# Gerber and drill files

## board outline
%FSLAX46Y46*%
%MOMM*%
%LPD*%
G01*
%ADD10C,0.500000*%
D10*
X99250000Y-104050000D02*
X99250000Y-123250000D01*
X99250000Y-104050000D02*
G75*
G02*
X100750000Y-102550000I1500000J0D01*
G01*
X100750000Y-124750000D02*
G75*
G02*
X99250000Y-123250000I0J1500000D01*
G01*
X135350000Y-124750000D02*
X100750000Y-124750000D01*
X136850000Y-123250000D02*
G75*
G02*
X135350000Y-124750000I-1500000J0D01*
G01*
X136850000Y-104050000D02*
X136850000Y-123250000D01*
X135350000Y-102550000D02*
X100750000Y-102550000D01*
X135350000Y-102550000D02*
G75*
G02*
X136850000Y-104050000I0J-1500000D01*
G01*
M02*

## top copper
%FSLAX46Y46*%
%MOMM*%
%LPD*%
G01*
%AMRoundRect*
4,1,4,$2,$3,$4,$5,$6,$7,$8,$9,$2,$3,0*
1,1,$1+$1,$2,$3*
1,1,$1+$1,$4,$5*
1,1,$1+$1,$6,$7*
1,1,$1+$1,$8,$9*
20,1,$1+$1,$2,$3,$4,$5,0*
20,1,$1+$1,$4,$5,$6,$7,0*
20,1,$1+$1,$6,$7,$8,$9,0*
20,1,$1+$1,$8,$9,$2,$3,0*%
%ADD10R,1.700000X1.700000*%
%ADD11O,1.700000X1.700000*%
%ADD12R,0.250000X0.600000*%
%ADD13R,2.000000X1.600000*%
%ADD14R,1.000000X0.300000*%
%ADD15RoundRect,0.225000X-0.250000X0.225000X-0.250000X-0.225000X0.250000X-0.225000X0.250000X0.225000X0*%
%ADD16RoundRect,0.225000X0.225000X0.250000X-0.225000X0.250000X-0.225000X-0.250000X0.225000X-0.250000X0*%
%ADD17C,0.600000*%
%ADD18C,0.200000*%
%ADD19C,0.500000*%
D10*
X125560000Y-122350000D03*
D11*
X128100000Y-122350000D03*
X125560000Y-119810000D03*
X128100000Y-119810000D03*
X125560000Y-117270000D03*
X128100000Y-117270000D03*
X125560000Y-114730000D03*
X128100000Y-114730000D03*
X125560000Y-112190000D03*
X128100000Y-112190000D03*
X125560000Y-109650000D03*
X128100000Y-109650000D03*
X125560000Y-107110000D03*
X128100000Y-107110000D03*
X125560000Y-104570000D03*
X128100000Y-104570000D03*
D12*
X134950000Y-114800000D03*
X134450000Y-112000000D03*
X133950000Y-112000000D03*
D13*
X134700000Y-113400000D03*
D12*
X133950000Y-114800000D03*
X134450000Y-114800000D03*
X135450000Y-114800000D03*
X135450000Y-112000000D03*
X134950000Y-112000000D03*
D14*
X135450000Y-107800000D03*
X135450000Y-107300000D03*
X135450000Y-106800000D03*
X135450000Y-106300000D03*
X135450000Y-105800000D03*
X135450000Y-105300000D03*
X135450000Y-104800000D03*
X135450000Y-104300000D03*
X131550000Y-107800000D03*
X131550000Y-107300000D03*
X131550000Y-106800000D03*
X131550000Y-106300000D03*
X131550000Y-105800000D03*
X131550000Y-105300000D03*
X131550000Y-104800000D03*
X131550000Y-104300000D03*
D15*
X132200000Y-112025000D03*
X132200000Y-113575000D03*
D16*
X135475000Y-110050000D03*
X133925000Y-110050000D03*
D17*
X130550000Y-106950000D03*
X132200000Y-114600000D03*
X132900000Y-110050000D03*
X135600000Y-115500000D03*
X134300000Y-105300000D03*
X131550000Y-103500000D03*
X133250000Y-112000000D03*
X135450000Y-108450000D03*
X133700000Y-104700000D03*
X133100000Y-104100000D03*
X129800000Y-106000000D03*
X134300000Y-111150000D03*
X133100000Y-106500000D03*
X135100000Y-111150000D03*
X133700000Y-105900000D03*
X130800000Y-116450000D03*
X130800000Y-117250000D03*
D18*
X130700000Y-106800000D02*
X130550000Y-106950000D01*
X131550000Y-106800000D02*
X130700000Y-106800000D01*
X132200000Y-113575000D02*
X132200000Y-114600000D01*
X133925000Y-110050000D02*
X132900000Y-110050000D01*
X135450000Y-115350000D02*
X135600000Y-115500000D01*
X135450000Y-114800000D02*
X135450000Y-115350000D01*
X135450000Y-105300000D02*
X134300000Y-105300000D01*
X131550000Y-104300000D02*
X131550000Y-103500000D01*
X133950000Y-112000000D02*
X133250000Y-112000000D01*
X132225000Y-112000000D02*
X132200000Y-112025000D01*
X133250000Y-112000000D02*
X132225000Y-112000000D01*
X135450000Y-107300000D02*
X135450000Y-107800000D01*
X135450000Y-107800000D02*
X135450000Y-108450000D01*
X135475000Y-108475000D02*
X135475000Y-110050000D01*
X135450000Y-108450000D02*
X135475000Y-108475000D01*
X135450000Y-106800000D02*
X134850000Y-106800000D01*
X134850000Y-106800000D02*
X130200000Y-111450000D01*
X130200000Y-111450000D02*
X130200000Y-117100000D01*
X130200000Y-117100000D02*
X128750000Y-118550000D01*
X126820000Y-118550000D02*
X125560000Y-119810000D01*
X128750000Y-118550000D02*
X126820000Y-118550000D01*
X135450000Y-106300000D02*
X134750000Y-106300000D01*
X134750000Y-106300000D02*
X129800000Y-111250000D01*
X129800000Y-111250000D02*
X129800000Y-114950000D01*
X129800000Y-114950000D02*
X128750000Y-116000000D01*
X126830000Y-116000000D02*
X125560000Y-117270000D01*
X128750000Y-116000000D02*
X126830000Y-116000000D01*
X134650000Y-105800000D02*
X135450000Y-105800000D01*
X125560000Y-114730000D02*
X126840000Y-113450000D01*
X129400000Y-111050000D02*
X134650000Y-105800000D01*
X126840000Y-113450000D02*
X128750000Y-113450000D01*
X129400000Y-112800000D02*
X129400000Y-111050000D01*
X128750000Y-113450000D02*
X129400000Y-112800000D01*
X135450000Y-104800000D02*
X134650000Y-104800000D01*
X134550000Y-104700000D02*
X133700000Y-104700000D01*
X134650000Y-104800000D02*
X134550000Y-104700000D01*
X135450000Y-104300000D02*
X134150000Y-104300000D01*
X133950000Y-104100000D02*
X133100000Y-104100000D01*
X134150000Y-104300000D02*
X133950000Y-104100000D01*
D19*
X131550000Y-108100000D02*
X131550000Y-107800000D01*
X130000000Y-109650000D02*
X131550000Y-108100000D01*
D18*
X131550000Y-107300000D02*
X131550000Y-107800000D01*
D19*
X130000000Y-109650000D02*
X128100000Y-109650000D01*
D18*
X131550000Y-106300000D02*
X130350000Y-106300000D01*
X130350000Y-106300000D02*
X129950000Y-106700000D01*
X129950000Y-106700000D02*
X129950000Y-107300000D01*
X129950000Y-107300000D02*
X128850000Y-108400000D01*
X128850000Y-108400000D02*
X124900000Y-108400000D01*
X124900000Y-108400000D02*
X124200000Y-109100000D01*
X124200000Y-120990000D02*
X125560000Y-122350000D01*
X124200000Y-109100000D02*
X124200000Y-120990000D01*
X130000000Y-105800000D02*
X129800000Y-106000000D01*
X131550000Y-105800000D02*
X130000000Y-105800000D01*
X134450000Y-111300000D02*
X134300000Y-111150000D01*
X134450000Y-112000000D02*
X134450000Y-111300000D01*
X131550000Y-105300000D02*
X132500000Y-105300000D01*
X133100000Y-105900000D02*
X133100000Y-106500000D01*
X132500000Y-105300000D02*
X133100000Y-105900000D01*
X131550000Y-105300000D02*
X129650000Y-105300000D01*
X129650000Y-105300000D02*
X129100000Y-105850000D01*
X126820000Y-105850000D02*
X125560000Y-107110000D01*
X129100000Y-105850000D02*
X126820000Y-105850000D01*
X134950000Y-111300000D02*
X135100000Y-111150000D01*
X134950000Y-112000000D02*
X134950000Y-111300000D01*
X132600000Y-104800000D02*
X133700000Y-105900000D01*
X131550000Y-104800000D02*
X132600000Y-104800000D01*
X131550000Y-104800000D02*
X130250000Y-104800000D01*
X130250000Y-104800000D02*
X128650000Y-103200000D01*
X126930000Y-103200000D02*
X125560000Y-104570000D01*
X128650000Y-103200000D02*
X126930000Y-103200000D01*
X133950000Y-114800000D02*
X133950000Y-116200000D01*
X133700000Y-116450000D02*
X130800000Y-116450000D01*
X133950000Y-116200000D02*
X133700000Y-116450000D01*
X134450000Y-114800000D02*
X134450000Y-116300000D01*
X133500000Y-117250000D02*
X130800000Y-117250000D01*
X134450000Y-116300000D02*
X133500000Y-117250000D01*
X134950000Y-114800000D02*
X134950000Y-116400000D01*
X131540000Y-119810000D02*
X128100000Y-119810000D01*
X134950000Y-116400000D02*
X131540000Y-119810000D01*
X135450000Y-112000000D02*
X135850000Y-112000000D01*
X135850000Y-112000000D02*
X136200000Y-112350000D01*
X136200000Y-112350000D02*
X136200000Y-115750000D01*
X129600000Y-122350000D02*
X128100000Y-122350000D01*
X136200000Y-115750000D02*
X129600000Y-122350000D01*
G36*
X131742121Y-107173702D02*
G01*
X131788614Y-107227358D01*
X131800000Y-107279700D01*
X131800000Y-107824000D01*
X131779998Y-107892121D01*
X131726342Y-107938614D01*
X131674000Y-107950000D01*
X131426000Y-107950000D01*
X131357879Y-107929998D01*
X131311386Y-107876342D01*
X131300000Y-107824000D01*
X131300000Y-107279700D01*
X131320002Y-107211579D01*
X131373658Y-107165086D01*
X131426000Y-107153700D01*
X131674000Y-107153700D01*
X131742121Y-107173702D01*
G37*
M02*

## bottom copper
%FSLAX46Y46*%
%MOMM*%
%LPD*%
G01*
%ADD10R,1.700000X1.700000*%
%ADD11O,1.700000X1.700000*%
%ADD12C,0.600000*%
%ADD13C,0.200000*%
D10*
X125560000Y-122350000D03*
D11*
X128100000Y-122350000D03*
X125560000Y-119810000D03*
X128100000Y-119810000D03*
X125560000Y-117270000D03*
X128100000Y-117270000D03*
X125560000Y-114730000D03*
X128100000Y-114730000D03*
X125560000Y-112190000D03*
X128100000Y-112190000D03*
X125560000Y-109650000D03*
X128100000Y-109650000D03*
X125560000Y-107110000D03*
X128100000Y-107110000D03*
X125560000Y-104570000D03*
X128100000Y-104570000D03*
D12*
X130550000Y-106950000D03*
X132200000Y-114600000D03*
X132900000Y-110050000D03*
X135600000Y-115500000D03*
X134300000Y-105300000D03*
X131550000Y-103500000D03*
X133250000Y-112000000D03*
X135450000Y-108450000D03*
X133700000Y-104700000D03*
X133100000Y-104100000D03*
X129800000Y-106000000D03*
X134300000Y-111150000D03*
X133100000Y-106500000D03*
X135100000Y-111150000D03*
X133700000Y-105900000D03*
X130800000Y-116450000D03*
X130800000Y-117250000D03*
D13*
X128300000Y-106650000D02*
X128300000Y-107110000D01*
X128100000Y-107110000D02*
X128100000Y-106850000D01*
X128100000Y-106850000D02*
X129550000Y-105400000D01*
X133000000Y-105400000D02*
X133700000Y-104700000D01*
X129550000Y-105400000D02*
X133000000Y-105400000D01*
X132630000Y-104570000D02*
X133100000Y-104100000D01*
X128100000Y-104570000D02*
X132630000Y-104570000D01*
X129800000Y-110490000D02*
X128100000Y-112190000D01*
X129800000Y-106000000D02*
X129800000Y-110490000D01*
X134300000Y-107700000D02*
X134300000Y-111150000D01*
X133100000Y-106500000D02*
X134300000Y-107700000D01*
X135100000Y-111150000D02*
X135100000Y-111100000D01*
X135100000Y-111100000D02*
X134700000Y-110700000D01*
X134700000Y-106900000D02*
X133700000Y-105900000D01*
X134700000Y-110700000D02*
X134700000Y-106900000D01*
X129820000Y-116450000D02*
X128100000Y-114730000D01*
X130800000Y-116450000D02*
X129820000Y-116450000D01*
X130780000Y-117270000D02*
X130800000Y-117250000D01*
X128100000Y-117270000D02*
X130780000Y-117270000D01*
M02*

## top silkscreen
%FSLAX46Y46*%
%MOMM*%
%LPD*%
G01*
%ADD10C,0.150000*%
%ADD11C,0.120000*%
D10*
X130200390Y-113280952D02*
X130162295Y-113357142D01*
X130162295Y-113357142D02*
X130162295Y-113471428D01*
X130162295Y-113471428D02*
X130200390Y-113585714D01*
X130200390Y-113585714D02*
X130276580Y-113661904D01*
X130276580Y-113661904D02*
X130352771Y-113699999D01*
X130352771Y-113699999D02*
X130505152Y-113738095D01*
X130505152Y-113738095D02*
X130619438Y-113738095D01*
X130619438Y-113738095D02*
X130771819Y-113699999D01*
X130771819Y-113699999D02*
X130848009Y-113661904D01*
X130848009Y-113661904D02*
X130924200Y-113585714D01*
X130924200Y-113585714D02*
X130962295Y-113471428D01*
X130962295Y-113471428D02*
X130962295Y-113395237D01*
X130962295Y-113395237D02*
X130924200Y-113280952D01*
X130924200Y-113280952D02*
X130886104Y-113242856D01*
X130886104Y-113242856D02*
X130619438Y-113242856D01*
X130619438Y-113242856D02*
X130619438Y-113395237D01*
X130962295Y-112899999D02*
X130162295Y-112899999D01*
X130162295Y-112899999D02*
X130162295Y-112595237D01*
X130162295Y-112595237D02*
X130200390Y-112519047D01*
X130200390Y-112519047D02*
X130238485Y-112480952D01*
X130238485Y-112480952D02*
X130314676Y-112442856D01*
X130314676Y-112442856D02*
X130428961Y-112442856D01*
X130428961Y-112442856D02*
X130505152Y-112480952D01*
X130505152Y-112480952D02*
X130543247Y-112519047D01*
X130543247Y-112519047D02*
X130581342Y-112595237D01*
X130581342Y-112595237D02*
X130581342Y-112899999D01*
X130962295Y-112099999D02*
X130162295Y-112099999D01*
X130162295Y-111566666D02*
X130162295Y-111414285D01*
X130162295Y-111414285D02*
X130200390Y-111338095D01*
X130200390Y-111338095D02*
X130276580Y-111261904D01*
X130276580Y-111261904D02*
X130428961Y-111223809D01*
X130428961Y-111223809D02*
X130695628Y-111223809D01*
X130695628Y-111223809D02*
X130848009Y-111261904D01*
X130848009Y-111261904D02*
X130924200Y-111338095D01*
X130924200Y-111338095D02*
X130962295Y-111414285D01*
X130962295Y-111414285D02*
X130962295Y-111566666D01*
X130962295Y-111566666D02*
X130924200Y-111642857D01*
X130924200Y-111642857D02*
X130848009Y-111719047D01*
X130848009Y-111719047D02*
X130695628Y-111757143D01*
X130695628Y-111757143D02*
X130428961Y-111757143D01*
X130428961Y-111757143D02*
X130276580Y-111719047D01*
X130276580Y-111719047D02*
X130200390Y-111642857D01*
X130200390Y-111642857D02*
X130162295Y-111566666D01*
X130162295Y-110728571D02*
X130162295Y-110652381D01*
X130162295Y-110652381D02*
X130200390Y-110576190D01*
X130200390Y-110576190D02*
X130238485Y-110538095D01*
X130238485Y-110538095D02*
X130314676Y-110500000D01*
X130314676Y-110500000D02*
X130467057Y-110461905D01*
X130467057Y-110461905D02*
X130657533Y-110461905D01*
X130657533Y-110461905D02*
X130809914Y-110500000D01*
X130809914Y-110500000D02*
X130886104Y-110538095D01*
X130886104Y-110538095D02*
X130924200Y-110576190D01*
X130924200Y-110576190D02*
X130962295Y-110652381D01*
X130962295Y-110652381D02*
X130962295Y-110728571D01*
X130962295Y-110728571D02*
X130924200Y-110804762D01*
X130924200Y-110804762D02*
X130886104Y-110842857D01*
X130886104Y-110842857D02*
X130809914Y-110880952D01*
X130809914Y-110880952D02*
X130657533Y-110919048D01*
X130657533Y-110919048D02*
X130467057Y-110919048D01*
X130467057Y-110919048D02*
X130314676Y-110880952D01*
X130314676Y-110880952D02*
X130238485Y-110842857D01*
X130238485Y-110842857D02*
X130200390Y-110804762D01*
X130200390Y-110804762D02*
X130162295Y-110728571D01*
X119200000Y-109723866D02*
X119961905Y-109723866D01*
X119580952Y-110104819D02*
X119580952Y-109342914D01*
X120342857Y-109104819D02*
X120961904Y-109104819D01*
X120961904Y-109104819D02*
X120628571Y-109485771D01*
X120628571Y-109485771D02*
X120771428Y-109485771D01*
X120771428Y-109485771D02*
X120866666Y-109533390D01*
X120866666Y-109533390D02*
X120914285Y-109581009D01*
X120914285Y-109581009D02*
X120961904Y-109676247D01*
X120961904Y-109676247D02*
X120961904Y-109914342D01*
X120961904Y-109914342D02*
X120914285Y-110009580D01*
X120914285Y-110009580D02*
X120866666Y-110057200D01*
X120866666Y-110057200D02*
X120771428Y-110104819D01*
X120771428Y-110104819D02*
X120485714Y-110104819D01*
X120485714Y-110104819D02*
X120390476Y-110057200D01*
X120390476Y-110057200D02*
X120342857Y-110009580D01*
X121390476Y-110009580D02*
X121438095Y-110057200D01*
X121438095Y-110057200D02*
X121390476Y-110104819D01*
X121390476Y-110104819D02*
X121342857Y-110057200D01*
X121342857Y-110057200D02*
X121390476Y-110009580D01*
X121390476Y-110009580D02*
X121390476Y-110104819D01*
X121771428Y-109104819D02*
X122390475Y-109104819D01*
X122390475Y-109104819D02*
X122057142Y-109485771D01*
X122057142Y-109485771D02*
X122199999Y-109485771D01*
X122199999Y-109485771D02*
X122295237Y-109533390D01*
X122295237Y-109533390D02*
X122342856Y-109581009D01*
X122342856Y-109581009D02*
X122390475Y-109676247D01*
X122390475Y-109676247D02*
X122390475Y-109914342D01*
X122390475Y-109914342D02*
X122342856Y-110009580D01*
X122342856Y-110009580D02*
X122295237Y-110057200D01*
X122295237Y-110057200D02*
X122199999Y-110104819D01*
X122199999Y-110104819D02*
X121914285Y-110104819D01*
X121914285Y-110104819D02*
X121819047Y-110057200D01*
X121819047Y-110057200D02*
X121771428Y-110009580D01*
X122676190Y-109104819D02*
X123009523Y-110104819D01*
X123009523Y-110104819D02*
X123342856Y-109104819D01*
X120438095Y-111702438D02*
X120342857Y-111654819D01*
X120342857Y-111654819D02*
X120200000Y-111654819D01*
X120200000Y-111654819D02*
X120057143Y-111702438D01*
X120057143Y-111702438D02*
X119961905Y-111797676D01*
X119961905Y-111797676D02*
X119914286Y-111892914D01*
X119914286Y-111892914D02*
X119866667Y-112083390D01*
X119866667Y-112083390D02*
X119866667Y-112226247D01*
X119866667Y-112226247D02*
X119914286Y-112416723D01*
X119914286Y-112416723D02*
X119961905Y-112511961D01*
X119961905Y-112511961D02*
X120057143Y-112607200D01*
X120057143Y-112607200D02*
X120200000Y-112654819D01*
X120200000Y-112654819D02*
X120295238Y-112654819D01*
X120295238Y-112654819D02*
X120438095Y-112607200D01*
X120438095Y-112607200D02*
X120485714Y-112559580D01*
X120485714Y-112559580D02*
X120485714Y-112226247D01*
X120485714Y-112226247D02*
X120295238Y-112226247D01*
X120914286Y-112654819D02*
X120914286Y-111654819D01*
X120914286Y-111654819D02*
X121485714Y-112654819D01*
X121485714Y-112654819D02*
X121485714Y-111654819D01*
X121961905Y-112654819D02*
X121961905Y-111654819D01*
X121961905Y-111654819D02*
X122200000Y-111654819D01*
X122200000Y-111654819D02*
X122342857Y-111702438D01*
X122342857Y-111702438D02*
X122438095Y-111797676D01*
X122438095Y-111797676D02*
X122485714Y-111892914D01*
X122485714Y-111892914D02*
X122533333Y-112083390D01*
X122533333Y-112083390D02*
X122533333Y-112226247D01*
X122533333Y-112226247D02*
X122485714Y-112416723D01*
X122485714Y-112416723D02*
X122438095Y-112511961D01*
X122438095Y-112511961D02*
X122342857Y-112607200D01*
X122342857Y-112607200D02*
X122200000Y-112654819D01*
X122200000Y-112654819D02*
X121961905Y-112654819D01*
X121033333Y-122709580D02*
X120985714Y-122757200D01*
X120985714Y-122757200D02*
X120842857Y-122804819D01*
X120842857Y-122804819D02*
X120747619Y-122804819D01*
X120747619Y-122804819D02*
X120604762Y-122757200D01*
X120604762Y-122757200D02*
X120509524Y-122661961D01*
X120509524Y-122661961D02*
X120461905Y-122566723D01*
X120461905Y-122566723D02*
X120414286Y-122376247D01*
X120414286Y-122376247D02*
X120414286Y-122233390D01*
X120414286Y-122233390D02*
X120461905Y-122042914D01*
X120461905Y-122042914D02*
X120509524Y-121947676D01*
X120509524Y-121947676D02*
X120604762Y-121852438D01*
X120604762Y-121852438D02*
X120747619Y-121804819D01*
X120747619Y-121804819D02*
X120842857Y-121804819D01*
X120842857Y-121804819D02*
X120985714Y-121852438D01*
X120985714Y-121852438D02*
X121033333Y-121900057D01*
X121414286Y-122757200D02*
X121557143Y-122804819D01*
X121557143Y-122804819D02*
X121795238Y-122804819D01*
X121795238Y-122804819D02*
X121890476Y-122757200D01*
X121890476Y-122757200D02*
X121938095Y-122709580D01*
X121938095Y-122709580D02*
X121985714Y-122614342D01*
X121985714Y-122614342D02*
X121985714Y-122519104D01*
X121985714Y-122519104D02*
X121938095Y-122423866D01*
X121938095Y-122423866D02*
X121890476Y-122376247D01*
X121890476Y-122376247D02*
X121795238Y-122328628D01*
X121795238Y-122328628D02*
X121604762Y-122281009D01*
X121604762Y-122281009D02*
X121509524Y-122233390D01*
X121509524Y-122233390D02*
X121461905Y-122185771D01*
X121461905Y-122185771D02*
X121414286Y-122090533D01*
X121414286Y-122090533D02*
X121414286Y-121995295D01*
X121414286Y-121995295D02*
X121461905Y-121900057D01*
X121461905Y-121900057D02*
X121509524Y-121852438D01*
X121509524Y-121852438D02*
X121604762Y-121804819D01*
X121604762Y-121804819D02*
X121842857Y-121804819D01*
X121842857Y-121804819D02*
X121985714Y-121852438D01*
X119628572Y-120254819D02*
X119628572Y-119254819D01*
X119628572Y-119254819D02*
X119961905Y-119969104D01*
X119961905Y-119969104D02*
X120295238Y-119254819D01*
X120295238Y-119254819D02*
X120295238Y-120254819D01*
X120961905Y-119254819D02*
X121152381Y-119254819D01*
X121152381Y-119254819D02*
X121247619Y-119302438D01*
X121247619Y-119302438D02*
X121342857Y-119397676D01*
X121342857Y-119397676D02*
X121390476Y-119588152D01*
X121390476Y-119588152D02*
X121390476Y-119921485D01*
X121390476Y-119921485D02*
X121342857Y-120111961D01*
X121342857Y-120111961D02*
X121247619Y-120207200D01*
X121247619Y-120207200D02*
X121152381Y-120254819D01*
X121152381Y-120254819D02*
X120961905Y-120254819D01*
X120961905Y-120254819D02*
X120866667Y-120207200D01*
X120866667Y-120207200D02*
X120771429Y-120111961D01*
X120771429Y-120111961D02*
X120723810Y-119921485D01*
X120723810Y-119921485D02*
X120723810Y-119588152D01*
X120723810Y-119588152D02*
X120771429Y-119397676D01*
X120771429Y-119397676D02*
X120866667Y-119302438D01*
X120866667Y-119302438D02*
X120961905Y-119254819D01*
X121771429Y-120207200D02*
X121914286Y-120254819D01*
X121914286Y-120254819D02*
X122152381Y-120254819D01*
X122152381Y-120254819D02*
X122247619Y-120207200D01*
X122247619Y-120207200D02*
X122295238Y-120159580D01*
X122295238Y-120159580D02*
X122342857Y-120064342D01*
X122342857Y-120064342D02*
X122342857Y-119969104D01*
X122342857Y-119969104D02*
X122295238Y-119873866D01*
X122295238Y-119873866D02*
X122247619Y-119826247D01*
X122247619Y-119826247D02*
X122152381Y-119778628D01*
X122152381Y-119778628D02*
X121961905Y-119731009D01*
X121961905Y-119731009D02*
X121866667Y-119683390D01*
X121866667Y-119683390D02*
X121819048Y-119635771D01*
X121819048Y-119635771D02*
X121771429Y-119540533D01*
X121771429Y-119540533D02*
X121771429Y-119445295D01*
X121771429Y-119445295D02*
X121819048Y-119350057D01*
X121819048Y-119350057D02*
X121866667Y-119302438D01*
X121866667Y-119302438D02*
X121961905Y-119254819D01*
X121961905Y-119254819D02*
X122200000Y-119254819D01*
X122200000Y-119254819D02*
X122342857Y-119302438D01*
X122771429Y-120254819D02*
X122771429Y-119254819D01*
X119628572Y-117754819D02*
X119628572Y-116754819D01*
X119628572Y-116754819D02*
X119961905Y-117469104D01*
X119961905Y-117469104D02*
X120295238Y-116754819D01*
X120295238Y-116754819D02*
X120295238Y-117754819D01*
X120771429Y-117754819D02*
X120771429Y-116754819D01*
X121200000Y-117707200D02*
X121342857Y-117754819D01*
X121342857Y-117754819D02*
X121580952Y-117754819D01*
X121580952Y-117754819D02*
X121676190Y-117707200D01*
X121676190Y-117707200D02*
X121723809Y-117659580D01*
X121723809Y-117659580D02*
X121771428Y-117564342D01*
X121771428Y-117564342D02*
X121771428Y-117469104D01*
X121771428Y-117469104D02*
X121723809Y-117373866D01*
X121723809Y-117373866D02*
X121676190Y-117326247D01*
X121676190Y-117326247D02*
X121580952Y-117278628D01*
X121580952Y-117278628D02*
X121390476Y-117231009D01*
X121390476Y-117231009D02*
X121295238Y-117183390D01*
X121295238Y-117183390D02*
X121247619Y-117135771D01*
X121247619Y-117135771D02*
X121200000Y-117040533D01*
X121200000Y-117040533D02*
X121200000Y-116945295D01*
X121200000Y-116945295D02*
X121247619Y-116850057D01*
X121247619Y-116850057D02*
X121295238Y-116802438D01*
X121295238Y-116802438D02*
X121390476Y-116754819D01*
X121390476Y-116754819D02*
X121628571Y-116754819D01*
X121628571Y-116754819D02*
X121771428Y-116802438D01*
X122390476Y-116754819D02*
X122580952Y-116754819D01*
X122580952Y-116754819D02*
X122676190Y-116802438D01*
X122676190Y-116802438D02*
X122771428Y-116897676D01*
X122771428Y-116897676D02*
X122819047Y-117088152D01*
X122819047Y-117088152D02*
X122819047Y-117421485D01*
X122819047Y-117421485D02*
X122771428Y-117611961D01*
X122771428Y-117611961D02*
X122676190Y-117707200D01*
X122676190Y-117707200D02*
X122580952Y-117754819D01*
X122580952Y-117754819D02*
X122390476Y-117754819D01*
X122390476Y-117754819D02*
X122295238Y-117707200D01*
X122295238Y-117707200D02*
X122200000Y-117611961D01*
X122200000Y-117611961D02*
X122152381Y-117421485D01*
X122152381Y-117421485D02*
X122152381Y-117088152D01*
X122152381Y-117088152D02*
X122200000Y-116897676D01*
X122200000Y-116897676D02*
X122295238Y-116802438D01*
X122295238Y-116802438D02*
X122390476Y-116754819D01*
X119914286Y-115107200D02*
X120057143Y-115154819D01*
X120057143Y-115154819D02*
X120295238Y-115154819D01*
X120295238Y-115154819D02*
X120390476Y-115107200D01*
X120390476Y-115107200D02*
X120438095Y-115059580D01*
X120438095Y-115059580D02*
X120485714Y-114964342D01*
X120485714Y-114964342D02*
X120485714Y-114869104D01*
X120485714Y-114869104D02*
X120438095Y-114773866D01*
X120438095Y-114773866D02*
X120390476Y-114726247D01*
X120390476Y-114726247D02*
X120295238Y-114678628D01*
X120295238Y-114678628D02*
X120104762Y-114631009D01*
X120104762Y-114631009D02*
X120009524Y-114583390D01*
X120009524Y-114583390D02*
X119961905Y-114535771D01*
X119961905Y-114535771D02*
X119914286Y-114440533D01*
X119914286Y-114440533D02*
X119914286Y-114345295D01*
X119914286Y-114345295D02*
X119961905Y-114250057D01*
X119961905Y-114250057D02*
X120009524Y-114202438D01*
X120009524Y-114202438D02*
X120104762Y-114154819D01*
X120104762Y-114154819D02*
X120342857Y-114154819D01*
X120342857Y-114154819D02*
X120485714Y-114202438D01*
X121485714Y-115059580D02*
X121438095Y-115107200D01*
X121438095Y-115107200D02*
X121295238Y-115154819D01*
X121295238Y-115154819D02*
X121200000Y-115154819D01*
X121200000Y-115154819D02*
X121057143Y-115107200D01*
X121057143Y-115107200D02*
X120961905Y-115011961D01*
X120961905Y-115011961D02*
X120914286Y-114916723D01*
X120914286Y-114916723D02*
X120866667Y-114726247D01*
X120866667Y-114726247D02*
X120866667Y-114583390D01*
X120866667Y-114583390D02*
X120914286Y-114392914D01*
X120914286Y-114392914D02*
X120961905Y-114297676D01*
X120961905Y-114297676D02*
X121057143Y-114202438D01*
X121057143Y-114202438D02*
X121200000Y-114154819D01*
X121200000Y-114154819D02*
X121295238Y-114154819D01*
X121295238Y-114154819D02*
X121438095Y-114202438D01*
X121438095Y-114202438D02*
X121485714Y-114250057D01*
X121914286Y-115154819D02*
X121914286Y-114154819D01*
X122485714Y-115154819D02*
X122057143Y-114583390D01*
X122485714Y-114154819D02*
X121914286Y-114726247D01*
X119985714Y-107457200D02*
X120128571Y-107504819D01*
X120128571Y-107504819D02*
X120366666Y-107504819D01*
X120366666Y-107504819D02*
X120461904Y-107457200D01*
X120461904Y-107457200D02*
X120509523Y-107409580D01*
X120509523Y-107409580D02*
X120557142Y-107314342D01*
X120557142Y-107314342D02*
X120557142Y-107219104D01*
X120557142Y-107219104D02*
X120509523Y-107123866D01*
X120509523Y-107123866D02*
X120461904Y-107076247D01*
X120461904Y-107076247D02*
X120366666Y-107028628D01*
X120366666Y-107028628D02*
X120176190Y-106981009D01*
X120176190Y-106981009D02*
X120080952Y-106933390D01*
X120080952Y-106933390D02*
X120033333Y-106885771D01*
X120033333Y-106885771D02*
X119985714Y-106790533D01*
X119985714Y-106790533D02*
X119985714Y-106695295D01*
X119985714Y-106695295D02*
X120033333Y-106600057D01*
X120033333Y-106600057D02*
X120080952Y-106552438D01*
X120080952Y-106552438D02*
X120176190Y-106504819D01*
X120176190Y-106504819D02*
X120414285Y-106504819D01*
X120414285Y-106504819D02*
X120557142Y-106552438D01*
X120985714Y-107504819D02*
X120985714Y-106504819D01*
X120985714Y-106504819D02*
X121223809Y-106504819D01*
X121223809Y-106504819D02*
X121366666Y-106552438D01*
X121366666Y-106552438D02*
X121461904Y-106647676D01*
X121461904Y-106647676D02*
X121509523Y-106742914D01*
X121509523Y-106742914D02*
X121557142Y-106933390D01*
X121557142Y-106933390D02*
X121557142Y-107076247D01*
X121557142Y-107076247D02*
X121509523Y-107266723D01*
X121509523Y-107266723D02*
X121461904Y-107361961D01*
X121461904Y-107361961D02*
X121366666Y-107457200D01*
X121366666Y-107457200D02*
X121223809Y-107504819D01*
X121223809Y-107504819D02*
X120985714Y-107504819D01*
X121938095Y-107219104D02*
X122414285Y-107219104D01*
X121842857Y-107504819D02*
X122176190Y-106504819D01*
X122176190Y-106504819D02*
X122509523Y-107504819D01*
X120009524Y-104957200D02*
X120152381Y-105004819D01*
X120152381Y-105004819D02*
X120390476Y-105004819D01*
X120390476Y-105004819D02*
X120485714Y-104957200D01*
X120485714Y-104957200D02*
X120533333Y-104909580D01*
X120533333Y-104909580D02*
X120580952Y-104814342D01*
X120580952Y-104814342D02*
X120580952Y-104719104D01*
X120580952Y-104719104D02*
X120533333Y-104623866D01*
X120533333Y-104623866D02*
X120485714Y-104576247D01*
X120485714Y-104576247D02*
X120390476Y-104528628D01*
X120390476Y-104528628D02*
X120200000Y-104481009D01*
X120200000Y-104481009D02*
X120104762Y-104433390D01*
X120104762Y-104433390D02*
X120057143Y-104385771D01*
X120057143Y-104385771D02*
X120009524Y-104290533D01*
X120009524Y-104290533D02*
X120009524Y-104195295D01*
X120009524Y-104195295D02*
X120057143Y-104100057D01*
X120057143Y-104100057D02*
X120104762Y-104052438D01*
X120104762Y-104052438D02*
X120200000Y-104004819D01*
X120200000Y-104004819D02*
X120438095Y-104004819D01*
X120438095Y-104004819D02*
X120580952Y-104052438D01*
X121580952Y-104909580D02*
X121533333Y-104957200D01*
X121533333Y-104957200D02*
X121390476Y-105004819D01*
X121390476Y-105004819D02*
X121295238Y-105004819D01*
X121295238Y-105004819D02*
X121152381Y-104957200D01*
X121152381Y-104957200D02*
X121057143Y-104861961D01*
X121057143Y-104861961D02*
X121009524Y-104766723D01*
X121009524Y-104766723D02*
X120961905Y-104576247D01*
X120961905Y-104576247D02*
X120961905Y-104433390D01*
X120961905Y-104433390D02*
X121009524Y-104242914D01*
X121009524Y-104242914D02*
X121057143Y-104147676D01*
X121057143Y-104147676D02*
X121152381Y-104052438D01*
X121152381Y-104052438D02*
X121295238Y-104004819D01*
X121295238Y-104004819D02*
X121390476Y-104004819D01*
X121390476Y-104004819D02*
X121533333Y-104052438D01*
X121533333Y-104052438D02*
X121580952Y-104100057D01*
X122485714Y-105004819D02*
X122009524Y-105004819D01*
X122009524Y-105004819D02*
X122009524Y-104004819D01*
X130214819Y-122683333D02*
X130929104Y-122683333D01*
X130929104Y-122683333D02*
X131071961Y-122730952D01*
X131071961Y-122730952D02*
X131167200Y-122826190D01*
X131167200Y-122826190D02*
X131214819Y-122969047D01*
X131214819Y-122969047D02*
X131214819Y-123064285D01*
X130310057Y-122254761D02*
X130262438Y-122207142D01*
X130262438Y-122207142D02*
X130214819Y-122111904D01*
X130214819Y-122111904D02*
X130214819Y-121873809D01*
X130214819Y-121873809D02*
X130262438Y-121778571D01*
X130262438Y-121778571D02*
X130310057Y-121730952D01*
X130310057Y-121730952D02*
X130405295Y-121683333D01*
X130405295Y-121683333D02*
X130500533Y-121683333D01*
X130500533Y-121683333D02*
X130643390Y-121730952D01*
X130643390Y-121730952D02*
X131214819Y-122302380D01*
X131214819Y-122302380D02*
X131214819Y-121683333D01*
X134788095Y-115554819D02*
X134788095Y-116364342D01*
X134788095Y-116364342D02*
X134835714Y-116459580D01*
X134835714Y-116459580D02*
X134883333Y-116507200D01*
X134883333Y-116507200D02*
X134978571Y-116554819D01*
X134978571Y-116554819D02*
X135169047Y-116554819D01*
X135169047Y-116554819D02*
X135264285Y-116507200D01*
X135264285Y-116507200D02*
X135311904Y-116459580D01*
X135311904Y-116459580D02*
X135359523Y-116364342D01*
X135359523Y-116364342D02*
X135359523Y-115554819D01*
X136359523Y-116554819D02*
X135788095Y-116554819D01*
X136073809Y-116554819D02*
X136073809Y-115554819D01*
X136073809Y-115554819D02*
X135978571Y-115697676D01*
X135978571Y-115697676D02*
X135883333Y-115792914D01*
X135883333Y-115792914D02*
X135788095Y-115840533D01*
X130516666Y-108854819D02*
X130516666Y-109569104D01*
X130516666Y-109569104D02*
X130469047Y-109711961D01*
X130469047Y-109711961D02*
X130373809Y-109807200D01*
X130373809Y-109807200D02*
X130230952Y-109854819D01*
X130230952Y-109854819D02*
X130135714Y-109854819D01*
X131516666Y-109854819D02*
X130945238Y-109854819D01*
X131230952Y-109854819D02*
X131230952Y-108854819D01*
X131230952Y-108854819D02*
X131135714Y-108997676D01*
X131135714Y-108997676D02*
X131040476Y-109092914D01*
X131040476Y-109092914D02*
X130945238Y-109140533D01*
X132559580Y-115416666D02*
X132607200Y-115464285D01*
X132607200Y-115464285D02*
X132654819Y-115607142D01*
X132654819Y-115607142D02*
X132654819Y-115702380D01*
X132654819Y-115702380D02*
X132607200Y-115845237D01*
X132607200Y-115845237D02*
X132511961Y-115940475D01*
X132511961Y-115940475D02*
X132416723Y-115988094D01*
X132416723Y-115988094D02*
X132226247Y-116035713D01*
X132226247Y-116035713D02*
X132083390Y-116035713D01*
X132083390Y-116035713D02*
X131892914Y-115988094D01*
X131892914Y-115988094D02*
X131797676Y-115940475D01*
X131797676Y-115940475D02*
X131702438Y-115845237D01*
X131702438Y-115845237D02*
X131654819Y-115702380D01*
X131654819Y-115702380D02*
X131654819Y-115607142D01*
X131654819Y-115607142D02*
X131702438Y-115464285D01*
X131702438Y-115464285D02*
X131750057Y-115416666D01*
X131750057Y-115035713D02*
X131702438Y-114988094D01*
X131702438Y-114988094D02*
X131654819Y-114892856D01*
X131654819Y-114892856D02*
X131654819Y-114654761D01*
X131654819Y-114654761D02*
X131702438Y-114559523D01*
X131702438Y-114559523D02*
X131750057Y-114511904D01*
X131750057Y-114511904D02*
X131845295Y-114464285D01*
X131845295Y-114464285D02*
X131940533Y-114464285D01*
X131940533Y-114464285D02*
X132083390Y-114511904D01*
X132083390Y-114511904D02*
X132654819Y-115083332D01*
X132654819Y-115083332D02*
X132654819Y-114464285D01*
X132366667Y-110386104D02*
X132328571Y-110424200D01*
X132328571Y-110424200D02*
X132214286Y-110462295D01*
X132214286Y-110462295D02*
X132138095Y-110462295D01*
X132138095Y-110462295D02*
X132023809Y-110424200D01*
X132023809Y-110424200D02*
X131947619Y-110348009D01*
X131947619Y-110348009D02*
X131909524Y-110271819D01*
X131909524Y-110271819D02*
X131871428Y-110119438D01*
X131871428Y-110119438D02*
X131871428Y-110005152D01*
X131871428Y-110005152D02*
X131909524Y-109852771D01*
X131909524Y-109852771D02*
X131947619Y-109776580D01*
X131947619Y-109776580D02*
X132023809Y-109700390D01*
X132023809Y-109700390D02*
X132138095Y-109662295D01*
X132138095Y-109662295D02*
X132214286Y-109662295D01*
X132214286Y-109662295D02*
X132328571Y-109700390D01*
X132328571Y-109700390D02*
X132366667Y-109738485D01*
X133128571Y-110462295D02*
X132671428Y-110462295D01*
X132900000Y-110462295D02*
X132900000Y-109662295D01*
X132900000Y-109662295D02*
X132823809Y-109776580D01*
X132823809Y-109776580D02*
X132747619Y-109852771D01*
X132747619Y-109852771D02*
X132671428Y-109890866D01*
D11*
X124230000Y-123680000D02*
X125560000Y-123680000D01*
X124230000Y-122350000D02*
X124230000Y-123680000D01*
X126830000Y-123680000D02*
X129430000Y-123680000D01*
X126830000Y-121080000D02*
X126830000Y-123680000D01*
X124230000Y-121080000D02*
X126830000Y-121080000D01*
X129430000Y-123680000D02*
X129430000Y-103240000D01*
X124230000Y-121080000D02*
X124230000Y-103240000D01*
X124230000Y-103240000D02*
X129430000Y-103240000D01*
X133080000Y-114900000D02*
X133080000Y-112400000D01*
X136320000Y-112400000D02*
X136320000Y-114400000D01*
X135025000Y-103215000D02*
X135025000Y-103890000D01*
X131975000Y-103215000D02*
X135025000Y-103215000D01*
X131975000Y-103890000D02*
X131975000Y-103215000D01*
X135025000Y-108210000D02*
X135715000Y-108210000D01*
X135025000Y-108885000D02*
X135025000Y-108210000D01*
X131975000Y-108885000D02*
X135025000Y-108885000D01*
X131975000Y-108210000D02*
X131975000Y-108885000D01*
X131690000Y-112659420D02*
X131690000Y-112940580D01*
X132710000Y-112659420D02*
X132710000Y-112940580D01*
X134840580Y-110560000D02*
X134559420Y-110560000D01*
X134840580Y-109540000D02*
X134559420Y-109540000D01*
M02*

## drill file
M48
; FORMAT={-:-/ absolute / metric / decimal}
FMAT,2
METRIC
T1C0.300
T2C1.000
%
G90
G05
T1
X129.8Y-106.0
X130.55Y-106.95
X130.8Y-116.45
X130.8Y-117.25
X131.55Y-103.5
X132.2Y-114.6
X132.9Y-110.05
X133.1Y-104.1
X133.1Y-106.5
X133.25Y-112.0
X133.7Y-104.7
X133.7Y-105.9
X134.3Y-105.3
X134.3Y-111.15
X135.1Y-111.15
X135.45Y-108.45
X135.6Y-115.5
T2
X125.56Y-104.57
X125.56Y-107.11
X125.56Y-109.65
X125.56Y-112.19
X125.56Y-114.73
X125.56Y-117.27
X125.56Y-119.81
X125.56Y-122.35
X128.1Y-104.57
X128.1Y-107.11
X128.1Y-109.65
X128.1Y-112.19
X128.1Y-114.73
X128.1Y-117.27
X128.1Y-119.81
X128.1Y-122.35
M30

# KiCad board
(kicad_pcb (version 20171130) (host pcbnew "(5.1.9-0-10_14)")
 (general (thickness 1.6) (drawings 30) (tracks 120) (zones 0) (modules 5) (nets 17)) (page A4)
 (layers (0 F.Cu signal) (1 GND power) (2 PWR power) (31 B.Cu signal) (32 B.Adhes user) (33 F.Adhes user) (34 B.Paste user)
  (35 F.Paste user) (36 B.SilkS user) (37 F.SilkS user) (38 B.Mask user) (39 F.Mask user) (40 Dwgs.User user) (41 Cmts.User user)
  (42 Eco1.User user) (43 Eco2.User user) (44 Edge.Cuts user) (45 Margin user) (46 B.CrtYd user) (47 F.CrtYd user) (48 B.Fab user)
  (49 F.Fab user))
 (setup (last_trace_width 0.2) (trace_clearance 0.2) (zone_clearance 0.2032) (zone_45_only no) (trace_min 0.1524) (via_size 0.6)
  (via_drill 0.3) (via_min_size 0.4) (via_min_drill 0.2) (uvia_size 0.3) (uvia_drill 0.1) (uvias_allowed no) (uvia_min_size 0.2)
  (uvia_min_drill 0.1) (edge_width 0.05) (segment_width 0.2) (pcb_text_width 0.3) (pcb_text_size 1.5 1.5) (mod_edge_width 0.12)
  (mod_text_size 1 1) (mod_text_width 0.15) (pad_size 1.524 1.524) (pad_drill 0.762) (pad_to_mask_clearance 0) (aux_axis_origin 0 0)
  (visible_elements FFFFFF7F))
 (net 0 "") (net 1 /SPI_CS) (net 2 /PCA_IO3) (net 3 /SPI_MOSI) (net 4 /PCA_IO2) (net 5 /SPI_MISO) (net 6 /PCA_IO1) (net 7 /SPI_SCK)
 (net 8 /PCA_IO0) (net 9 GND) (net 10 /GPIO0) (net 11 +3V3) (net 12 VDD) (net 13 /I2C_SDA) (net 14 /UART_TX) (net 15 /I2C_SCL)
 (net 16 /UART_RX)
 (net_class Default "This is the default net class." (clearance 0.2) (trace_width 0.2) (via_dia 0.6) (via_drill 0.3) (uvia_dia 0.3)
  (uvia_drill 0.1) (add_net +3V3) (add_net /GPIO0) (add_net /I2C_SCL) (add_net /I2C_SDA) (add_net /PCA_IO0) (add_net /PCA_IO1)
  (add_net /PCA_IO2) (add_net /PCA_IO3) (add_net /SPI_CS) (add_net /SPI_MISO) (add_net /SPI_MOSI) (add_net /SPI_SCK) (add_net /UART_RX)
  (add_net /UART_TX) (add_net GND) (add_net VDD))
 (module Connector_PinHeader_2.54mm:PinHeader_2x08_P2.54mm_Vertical (layer F.Cu) (at 125.76 122.35 180)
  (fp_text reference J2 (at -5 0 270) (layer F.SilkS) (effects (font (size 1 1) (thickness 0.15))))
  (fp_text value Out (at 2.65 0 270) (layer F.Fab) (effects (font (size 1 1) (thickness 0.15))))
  (fp_line (start 1.53 -1.33) (end 0.2 -1.33) (layer F.SilkS) (width 0.12))
  (fp_line (start 1.53 0) (end 1.53 -1.33) (layer F.SilkS) (width 0.12))
  (fp_line (start -1.07 -1.33) (end -3.67 -1.33) (layer F.SilkS) (width 0.12))
  (fp_line (start -1.07 1.27) (end -1.07 -1.33) (layer F.SilkS) (width 0.12))
  (fp_line (start 1.53 1.27) (end -1.07 1.27) (layer F.SilkS) (width 0.12))
  (fp_line (start -3.67 -1.33) (end -3.67 19.11) (layer F.SilkS) (width 0.12))
  (fp_line (start 1.53 1.27) (end 1.53 19.11) (layer F.SilkS) (width 0.12))
  (fp_line (start 1.53 19.11) (end -3.67 19.11) (layer F.SilkS) (width 0.12))
  (pad 1 thru_hole rect (at 0.2 0 180) (size 1.7 1.7) (drill 1) (layers *.Cu *.Mask) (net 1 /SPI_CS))
  (pad 2 thru_hole oval (at -2.34 0 180) (size 1.7 1.7) (drill 1) (layers *.Cu *.Mask) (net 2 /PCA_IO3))
  (pad 3 thru_hole oval (at 0.2 2.54 180) (size 1.7 1.7) (drill 1) (layers *.Cu *.Mask) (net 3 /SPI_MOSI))
  (pad 4 thru_hole oval (at -2.34 2.54 180) (size 1.7 1.7) (drill 1) (layers *.Cu *.Mask) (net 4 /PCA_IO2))
  (pad 5 thru_hole oval (at 0.2 5.08 180) (size 1.7 1.7) (drill 1) (layers *.Cu *.Mask) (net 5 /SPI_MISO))
  (pad 6 thru_hole oval (at -2.34 5.08 180) (size 1.7 1.7) (drill 1) (layers *.Cu *.Mask) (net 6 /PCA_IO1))
  (pad 7 thru_hole oval (at 0.2 7.62 180) (size 1.7 1.7) (drill 1) (layers *.Cu *.Mask) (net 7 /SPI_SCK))
  (pad 8 thru_hole oval (at -2.34 7.62 180) (size 1.7 1.7) (drill 1) (layers *.Cu *.Mask) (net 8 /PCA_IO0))
  (pad 9 thru_hole oval (at 0.2 10.16 180) (size 1.7 1.7) (drill 1) (layers *.Cu *.Mask) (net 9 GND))
  (pad 10 thru_hole oval (at -2.34 10.16 180) (size 1.7 1.7) (drill 1) (layers *.Cu *.Mask) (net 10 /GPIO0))
  (pad 11 thru_hole oval (at 0.2 12.7 180) (size 1.7 1.7) (drill 1) (layers *.Cu *.Mask) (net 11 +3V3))
  (pad 12 thru_hole oval (at -2.34 12.7 180) (size 1.7 1.7) (drill 1) (layers *.Cu *.Mask) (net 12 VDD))
  (pad 13 thru_hole oval (at 0.2 15.24 180) (size 1.7 1.7) (drill 1) (layers *.Cu *.Mask) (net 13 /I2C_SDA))
  (pad 14 thru_hole oval (at -2.34 15.24 180) (size 1.7 1.7) (drill 1) (layers *.Cu *.Mask) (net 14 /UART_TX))
  (pad 15 thru_hole oval (at 0.2 17.78 180) (size 1.7 1.7) (drill 1) (layers *.Cu *.Mask) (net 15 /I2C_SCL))
  (pad 16 thru_hole oval (at -2.34 17.78 180) (size 1.7 1.7) (drill 1) (layers *.Cu *.Mask) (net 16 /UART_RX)))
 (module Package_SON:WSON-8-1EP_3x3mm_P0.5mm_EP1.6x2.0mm (layer F.Cu) (at 134.7 113.4 90)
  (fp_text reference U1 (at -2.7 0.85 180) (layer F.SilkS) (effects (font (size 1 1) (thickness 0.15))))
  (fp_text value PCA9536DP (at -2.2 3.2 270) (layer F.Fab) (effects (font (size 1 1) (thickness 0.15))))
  (fp_line (start -1.5 -1.62) (end 1 -1.62) (layer F.SilkS) (width 0.12))
  (fp_line (start 1 1.62) (end -1 1.62) (layer F.SilkS) (width 0.12))
  (pad 3 smd rect (at -1.4 0.25 90) (size 0.6 0.25) (layers F.Cu F.Paste F.Mask) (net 4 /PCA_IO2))
  (pad 7 smd rect (at 1.4 -0.25 90) (size 0.6 0.25) (layers F.Cu F.Paste F.Mask) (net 13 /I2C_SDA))
  (pad 8 smd rect (at 1.4 -0.75 90) (size 0.6 0.25) (layers F.Cu F.Paste F.Mask) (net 11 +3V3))
  (pad 9 smd rect (at 0 0 90) (size 1.6 2) (layers F.Cu F.Mask))
  (pad 1 smd rect (at -1.4 -0.75 90) (size 0.6 0.25) (layers F.Cu F.Paste F.Mask) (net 8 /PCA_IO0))
  (pad 2 smd rect (at -1.4 -0.25 90) (size 0.6 0.25) (layers F.Cu F.Paste F.Mask) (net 6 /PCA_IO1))
  (pad 4 smd rect (at -1.4 0.75 90) (size 0.6 0.25) (layers F.Cu F.Paste F.Mask) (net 9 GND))
  (pad 5 smd rect (at 1.4 0.75 90) (size 0.6 0.25) (layers F.Cu F.Paste F.Mask) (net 2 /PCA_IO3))
  (pad 6 smd rect (at 1.4 0.25 90) (size 0.6 0.25) (layers F.Cu F.Paste F.Mask) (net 15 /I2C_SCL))
  (pad "" smd rect (at -0.45 -0.55 90) (size 0.6 0.8) (layers F.Paste))
  (pad "" smd rect (at 0.45 -0.55 90) (size 0.6 0.8) (layers F.Paste))
  (pad "" smd rect (at -0.45 0.55 90) (size 0.6 0.8) (layers F.Paste))
  (pad "" smd rect (at 0.45 0.55 90) (size 0.6 0.8) (layers F.Paste)))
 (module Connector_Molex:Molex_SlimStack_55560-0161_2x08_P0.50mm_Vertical (layer F.Cu) (at 133.5 106.05 270)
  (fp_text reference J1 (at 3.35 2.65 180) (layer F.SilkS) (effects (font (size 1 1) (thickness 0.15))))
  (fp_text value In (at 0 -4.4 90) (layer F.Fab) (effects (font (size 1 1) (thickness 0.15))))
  (fp_line (start -2.835 -1.525) (end -2.16 -1.525) (layer F.SilkS) (width 0.12))
  (fp_line (start -2.835 1.525) (end -2.835 -1.525) (layer F.SilkS) (width 0.12))
  (fp_line (start -2.16 1.525) (end -2.835 1.525) (layer F.SilkS) (width 0.12))
  (fp_line (start 2.16 -1.525) (end 2.16 -2.215) (layer F.SilkS) (width 0.12))
  (fp_line (start 2.835 -1.525) (end 2.16 -1.525) (layer F.SilkS) (width 0.12))
  (fp_line (start 2.835 1.525) (end 2.835 -1.525) (layer F.SilkS) (width 0.12))
  (fp_line (start 2.16 1.525) (end 2.835 1.525) (layer F.SilkS) (width 0.12))
  (pad 1 smd rect (at 1.75 -1.95 270) (size 0.3 1) (layers F.Cu F.Paste F.Mask) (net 11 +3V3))
  (pad 3 smd rect (at 1.25 -1.95 270) (size 0.3 1) (layers F.Cu F.Paste F.Mask) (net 11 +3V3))
  (pad 5 smd rect (at 0.75 -1.95 270) (size 0.3 1) (layers F.Cu F.Paste F.Mask) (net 3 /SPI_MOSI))
  (pad 7 smd rect (at 0.25 -1.95 270) (size 0.3 1) (layers F.Cu F.Paste F.Mask) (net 5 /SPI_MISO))
  (pad 9 smd rect (at -0.25 -1.95 270) (size 0.3 1) (layers F.Cu F.Paste F.Mask) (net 7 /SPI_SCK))
  (pad 11 smd rect (at -0.75 -1.95 270) (size 0.3 1) (layers F.Cu F.Paste F.Mask) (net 9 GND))
  (pad 13 smd rect (at -1.25 -1.95 270) (size 0.3 1) (layers F.Cu F.Paste F.Mask) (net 14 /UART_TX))
  (pad 15 smd rect (at -1.75 -1.95 270) (size 0.3 1) (layers F.Cu F.Paste F.Mask) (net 16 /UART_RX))
  (pad 2 smd rect (at 1.75 1.95 270) (size 0.3 1) (layers F.Cu F.Paste F.Mask) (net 12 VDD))
  (pad 4 smd rect (at 1.25 1.95 270) (size 0.3 1) (layers F.Cu F.Paste F.Mask) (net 12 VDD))
  (pad 6 smd rect (at 0.75 1.95 270) (size 0.3 1) (layers F.Cu F.Paste F.Mask) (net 9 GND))
  (pad 8 smd rect (at 0.25 1.95 270) (size 0.3 1) (layers F.Cu F.Paste F.Mask) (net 1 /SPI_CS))
  (pad 10 smd rect (at -0.25 1.95 270) (size 0.3 1) (layers F.Cu F.Paste F.Mask) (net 10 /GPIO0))
  (pad 12 smd rect (at -0.75 1.95 270) (size 0.3 1) (layers F.Cu F.Paste F.Mask) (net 13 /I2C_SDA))
  (pad 14 smd rect (at -1.25 1.95 270) (size 0.3 1) (layers F.Cu F.Paste F.Mask) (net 15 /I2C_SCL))
  (pad 16 smd rect (at -1.75 1.95 270) (size 0.3 1) (layers F.Cu F.Paste F.Mask) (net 9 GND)))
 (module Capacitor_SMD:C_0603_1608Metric (layer F.Cu) (at 132.2 112.8 270)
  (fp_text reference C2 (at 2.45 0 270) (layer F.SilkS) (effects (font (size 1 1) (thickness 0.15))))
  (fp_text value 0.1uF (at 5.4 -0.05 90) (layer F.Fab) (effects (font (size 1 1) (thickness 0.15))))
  (fp_line (start -0.14058 0.51) (end 0.14058 0.51) (layer F.SilkS) (width 0.12))
  (fp_line (start -0.14058 -0.51) (end 0.14058 -0.51) (layer F.SilkS) (width 0.12))
  (pad 1 smd roundrect (at -0.775 0 270) (size 0.9 0.95) (layers F.Cu F.Paste F.Mask) (roundrect_rratio 0.25) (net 11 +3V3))
  (pad 2 smd roundrect (at 0.775 0 270) (size 0.9 0.95) (layers F.Cu F.Paste F.Mask) (roundrect_rratio 0.25) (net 9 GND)))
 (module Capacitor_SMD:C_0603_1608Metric (layer F.Cu) (at 134.7 110.05 180)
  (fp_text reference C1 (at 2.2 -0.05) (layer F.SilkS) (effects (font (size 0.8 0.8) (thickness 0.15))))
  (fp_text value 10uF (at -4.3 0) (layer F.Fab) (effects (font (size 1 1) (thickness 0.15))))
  (fp_line (start -0.14058 -0.51) (end 0.14058 -0.51) (layer F.SilkS) (width 0.12))
  (fp_line (start -0.14058 0.51) (end 0.14058 0.51) (layer F.SilkS) (width 0.12))
  (pad 1 smd roundrect (at -0.775 0 180) (size 0.9 0.95) (layers F.Cu F.Paste F.Mask) (roundrect_rratio 0.25) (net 11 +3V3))
  (pad 2 smd roundrect (at 0.775 0 180) (size 0.9 0.95) (layers F.Cu F.Paste F.Mask) (roundrect_rratio 0.25) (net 9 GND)))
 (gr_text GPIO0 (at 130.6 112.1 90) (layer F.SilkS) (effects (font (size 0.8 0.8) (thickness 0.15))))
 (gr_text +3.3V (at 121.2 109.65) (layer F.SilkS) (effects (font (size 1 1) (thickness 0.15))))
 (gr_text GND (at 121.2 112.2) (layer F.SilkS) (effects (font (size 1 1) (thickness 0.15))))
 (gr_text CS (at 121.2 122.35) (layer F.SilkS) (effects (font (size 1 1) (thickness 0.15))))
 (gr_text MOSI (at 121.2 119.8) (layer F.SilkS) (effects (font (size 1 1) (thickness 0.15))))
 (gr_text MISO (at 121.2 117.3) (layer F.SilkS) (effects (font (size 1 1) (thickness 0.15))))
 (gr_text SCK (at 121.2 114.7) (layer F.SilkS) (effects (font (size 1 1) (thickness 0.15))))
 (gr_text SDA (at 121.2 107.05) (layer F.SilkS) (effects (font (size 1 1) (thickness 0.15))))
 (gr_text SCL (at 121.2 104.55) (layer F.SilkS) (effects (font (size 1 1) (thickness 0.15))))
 (gr_line (start 99.25 104.05) (end 99.25 123.25) (layer Edge.Cuts) (width 0.5))
 (gr_arc (start 100.75 104.05) (end 99.25 104.05) (angle 90) (layer Edge.Cuts) (width 0.5))
 (gr_arc (start 100.75 123.25) (end 100.75 124.75) (angle 90) (layer Edge.Cuts) (width 0.5))
 (gr_line (start 135.35 124.75) (end 100.75 124.75) (layer Edge.Cuts) (width 0.5))
 (gr_arc (start 135.35 123.25) (end 136.85 123.25) (angle 90) (layer Edge.Cuts) (width 0.5))
 (gr_line (start 136.85 104.05) (end 136.85 123.25) (layer Edge.Cuts) (width 0.5))
 (gr_line (start 135.35 102.55) (end 100.75 102.55) (layer Edge.Cuts) (width 0.5))
 (gr_arc (start 135.35 104.05) (end 135.35 102.55) (angle 90) (layer Edge.Cuts) (width 0.5))
 (via (at 130.55 106.95) (size 0.6) (drill 0.3) (layers F.Cu B.Cu) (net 9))
 (segment (start 130.7 106.8) (end 130.55 106.95) (width 0.2) (layer F.Cu) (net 9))
 (segment (start 131.55 106.8) (end 130.7 106.8) (width 0.2) (layer F.Cu) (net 9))
 (via (at 132.2 114.6) (size 0.6) (drill 0.3) (layers F.Cu B.Cu) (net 9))
 (segment (start 132.2 113.575) (end 132.2 114.6) (width 0.2) (layer F.Cu) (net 9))
 (via (at 132.9 110.05) (size 0.6) (drill 0.3) (layers F.Cu B.Cu) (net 9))
 (segment (start 133.925 110.05) (end 132.9 110.05) (width 0.2) (layer F.Cu) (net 9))
 (via (at 135.6 115.5) (size 0.6) (drill 0.3) (layers F.Cu B.Cu) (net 9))
 (segment (start 135.45 115.35) (end 135.6 115.5) (width 0.2) (layer F.Cu) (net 9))
 (segment (start 135.45 114.8) (end 135.45 115.35) (width 0.2) (layer F.Cu) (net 9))
 (via (at 134.3 105.3) (size 0.6) (drill 0.3) (layers F.Cu B.Cu) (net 9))
 (segment (start 135.45 105.3) (end 134.3 105.3) (width 0.2) (layer F.Cu) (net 9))
 (via (at 131.55 103.5) (size 0.6) (drill 0.3) (layers F.Cu B.Cu) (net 9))
 (segment (start 131.55 104.3) (end 131.55 103.5) (width 0.2) (layer F.Cu) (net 9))
 (via (at 133.25 112) (size 0.6) (drill 0.3) (layers F.Cu B.Cu) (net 11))
 (segment (start 133.95 112) (end 133.25 112) (width 0.2) (layer F.Cu) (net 11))
 (segment (start 132.225 112) (end 132.2 112.025) (width 0.2) (layer F.Cu) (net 11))
 (segment (start 133.25 112) (end 132.225 112) (width 0.2) (layer F.Cu) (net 11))
 (segment (start 135.45 107.3) (end 135.45 107.8) (width 0.2) (layer F.Cu) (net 11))
 (via (at 135.45 108.45) (size 0.6) (drill 0.3) (layers F.Cu B.Cu) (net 11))
 (segment (start 135.45 107.8) (end 135.45 108.45) (width 0.2) (layer F.Cu) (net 11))
 (segment (start 135.475 108.475) (end 135.475 110.05) (width 0.2) (layer F.Cu) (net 11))
 (segment (start 135.45 108.45) (end 135.475 108.475) (width 0.2) (layer F.Cu) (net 11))
 (segment (start 135.45 106.8) (end 134.85 106.8) (width 0.2) (layer F.Cu) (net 3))
 (segment (start 134.85 106.8) (end 130.2 111.45) (width 0.2) (layer F.Cu) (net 3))
 (segment (start 130.2 111.45) (end 130.2 117.1) (width 0.2) (layer F.Cu) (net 3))
 (segment (start 130.2 117.1) (end 128.75 118.55) (width 0.2) (layer F.Cu) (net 3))
 (segment (start 126.82 118.55) (end 125.56 119.81) (width 0.2) (layer F.Cu) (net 3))
 (segment (start 128.75 118.55) (end 126.82 118.55) (width 0.2) (layer F.Cu) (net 3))
 (segment (start 135.45 106.3) (end 134.75 106.3) (width 0.2) (layer F.Cu) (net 5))
 (segment (start 134.75 106.3) (end 129.8 111.25) (width 0.2) (layer F.Cu) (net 5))
 (segment (start 129.8 111.25) (end 129.8 114.95) (width 0.2) (layer F.Cu) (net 5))
 (segment (start 129.8 114.95) (end 128.75 116) (width 0.2) (layer F.Cu) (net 5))
 (segment (start 126.83 116) (end 125.56 117.27) (width 0.2) (layer F.Cu) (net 5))
 (segment (start 128.75 116) (end 126.83 116) (width 0.2) (layer F.Cu) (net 5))
 (segment (start 134.65 105.8) (end 135.45 105.8) (width 0.2) (layer F.Cu) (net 7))
 (segment (start 125.56 114.73) (end 126.84 113.45) (width 0.2) (layer F.Cu) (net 7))
 (segment (start 129.4 111.05) (end 134.65 105.8) (width 0.2) (layer F.Cu) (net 7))
 (segment (start 126.84 113.45) (end 128.75 113.45) (width 0.2) (layer F.Cu) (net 7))
 (segment (start 129.4 112.8) (end 129.4 111.05) (width 0.2) (layer F.Cu) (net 7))
 (segment (start 128.75 113.45) (end 129.4 112.8) (width 0.2) (layer F.Cu) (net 7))
 (segment (start 135.45 104.8) (end 134.65 104.8) (width 0.2) (layer F.Cu) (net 14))
 (via (at 133.7 104.7) (size 0.6) (drill 0.3) (layers F.Cu B.Cu) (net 14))
 (segment (start 134.55 104.7) (end 133.7 104.7) (width 0.2) (layer F.Cu) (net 14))
 (segment (start 134.65 104.8) (end 134.55 104.7) (width 0.2) (layer F.Cu) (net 14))
 (segment (start 128.3 106.65) (end 128.3 107.11) (width 0.2) (layer B.Cu) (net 14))
 (segment (start 128.1 107.11) (end 128.1 106.85) (width 0.2) (layer B.Cu) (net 14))
 (segment (start 128.1 106.85) (end 129.55 105.4) (width 0.2) (layer B.Cu) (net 14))
 (segment (start 133 105.4) (end 133.7 104.7) (width 0.2) (layer B.Cu) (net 14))
 (segment (start 129.55 105.4) (end 133 105.4) (width 0.2) (layer B.Cu) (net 14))
 (segment (start 135.45 104.3) (end 134.15 104.3) (width 0.2) (layer F.Cu) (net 16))
 (via (at 133.1 104.1) (size 0.6) (drill 0.3) (layers F.Cu B.Cu) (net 16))
 (segment (start 133.95 104.1) (end 133.1 104.1) (width 0.2) (layer F.Cu) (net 16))
 (segment (start 134.15 104.3) (end 133.95 104.1) (width 0.2) (layer F.Cu) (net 16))
 (segment (start 132.63 104.57) (end 133.1 104.1) (width 0.2) (layer B.Cu) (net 16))
 (segment (start 128.1 104.57) (end 132.63 104.57) (width 0.2) (layer B.Cu) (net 16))
 (segment (start 131.55 108.1) (end 131.55 107.8) (width 0.5) (layer F.Cu) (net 12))
 (segment (start 130 109.65) (end 131.55 108.1) (width 0.5) (layer F.Cu) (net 12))
 (segment (start 131.55 107.3) (end 131.55 107.8) (width 0.2) (layer F.Cu) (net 12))
 (segment (start 130 109.65) (end 128.1 109.65) (width 0.5) (layer F.Cu) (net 12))
 (segment (start 131.55 106.3) (end 130.35 106.3) (width 0.2) (layer F.Cu) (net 1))
 (segment (start 130.35 106.3) (end 129.95 106.7) (width 0.2) (layer F.Cu) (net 1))
 (segment (start 129.95 106.7) (end 129.95 107.3) (width 0.2) (layer F.Cu) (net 1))
 (segment (start 129.95 107.3) (end 128.85 108.4) (width 0.2) (layer F.Cu) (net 1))
 (segment (start 128.85 108.4) (end 124.9 108.4) (width 0.2) (layer F.Cu) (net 1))
 (segment (start 124.9 108.4) (end 124.2 109.1) (width 0.2) (layer F.Cu) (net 1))
 (segment (start 124.2 120.99) (end 125.56 122.35) (width 0.2) (layer F.Cu) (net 1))
 (segment (start 124.2 109.1) (end 124.2 120.99) (width 0.2) (layer F.Cu) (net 1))
 (via (at 129.8 106) (size 0.6) (drill 0.3) (layers F.Cu B.Cu) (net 10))
 (segment (start 130 105.8) (end 129.8 106) (width 0.2) (layer F.Cu) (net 10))
 (segment (start 131.55 105.8) (end 130 105.8) (width 0.2) (layer F.Cu) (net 10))
 (segment (start 129.8 110.49) (end 128.1 112.19) (width 0.2) (layer B.Cu) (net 10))
 (segment (start 129.8 106) (end 129.8 110.49) (width 0.2) (layer B.Cu) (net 10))
 (via (at 134.3 111.15) (size 0.6) (drill 0.3) (layers F.Cu B.Cu) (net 13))
 (segment (start 134.45 111.3) (end 134.3 111.15) (width 0.2) (layer F.Cu) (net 13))
 (segment (start 134.45 112) (end 134.45 111.3) (width 0.2) (layer F.Cu) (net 13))
 (segment (start 131.55 105.3) (end 132.5 105.3) (width 0.2) (layer F.Cu) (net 13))
 (via (at 133.1 106.5) (size 0.6) (drill 0.3) (layers F.Cu B.Cu) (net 13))
 (segment (start 133.1 105.9) (end 133.1 106.5) (width 0.2) (layer F.Cu) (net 13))
 (segment (start 132.5 105.3) (end 133.1 105.9) (width 0.2) (layer F.Cu) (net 13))
 (segment (start 134.3 107.7) (end 134.3 111.15) (width 0.2) (layer B.Cu) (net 13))
 (segment (start 133.1 106.5) (end 134.3 107.7) (width 0.2) (layer B.Cu) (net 13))
 (segment (start 131.55 105.3) (end 129.65 105.3) (width 0.2) (layer F.Cu) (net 13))
 (segment (start 129.65 105.3) (end 129.1 105.85) (width 0.2) (layer F.Cu) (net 13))
 (segment (start 126.82 105.85) (end 125.56 107.11) (width 0.2) (layer F.Cu) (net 13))
 (segment (start 129.1 105.85) (end 126.82 105.85) (width 0.2) (layer F.Cu) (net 13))
 (via (at 135.1 111.15) (size 0.6) (drill 0.3) (layers F.Cu B.Cu) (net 15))
 (segment (start 134.95 111.3) (end 135.1 111.15) (width 0.2) (layer F.Cu) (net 15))
 (segment (start 134.95 112) (end 134.95 111.3) (width 0.2) (layer F.Cu) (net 15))
 (via (at 133.7 105.9) (size 0.6) (drill 0.3) (layers F.Cu B.Cu) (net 15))
 (segment (start 132.6 104.8) (end 133.7 105.9) (width 0.2) (layer F.Cu) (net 15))
 (segment (start 131.55 104.8) (end 132.6 104.8) (width 0.2) (layer F.Cu) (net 15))
 (segment (start 135.1 111.15) (end 135.1 111.1) (width 0.2) (layer B.Cu) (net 15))
 (segment (start 135.1 111.1) (end 134.7 110.7) (width 0.2) (layer B.Cu) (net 15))
 (segment (start 134.7 106.9) (end 133.7 105.9) (width 0.2) (layer B.Cu) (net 15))
 (segment (start 134.7 110.7) (end 134.7 106.9) (width 0.2) (layer B.Cu) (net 15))
 (segment (start 131.55 104.8) (end 130.25 104.8) (width 0.2) (layer F.Cu) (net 15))
 (segment (start 130.25 104.8) (end 128.65 103.2) (width 0.2) (layer F.Cu) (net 15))
 (segment (start 126.93 103.2) (end 125.56 104.57) (width 0.2) (layer F.Cu) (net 15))
 (segment (start 128.65 103.2) (end 126.93 103.2) (width 0.2) (layer F.Cu) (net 15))
 (segment (start 133.95 114.8) (end 133.95 116.2) (width 0.2) (layer F.Cu) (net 8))
 (via (at 130.8 116.45) (size 0.6) (drill 0.3) (layers F.Cu B.Cu) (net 8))
 (segment (start 133.7 116.45) (end 130.8 116.45) (width 0.2) (layer F.Cu) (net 8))
 (segment (start 133.95 116.2) (end 133.7 116.45) (width 0.2) (layer F.Cu) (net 8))
 (segment (start 129.82 116.45) (end 128.1 114.73) (width 0.2) (layer B.Cu) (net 8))
 (segment (start 130.8 116.45) (end 129.82 116.45) (width 0.2) (layer B.Cu) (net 8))
 (segment (start 134.45 114.8) (end 134.45 116.3) (width 0.2) (layer F.Cu) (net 6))
 (via (at 130.8 117.25) (size 0.6) (drill 0.3) (layers F.Cu B.Cu) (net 6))
 (segment (start 133.5 117.25) (end 130.8 117.25) (width 0.2) (layer F.Cu) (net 6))
 (segment (start 134.45 116.3) (end 133.5 117.25) (width 0.2) (layer F.Cu) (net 6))
 (segment (start 130.78 117.27) (end 130.8 117.25) (width 0.2) (layer B.Cu) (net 6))
 (segment (start 128.1 117.27) (end 130.78 117.27) (width 0.2) (layer B.Cu) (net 6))
 (segment (start 134.95 114.8) (end 134.95 116.4) (width 0.2) (layer F.Cu) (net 4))
 (segment (start 131.54 119.81) (end 128.1 119.81) (width 0.2) (layer F.Cu) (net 4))
 (segment (start 134.95 116.4) (end 131.54 119.81) (width 0.2) (layer F.Cu) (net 4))
 (segment (start 135.45 112) (end 135.85 112) (width 0.2) (layer F.Cu) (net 2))
 (segment (start 135.85 112) (end 136.2 112.35) (width 0.2) (layer F.Cu) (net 2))
 (segment (start 136.2 112.35) (end 136.2 115.75) (width 0.2) (layer F.Cu) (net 2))
 (segment (start 129.6 122.35) (end 128.1 122.35) (width 0.2) (layer F.Cu) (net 2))
 (segment (start 136.2 115.75) (end 129.6 122.35) (width 0.2) (layer F.Cu) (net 2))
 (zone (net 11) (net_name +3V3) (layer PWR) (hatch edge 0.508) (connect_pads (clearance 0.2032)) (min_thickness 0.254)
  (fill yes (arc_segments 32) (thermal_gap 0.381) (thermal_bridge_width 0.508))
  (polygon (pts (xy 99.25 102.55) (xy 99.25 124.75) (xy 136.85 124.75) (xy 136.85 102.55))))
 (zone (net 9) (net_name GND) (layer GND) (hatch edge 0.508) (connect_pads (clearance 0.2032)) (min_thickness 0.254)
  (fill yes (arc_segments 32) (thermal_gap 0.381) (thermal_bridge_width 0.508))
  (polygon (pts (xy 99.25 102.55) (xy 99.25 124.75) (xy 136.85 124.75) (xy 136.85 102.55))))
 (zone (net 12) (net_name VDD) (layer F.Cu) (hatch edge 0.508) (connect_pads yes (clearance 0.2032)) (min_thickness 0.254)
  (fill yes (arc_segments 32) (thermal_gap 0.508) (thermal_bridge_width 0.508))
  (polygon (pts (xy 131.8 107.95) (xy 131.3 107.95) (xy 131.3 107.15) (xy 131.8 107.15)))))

